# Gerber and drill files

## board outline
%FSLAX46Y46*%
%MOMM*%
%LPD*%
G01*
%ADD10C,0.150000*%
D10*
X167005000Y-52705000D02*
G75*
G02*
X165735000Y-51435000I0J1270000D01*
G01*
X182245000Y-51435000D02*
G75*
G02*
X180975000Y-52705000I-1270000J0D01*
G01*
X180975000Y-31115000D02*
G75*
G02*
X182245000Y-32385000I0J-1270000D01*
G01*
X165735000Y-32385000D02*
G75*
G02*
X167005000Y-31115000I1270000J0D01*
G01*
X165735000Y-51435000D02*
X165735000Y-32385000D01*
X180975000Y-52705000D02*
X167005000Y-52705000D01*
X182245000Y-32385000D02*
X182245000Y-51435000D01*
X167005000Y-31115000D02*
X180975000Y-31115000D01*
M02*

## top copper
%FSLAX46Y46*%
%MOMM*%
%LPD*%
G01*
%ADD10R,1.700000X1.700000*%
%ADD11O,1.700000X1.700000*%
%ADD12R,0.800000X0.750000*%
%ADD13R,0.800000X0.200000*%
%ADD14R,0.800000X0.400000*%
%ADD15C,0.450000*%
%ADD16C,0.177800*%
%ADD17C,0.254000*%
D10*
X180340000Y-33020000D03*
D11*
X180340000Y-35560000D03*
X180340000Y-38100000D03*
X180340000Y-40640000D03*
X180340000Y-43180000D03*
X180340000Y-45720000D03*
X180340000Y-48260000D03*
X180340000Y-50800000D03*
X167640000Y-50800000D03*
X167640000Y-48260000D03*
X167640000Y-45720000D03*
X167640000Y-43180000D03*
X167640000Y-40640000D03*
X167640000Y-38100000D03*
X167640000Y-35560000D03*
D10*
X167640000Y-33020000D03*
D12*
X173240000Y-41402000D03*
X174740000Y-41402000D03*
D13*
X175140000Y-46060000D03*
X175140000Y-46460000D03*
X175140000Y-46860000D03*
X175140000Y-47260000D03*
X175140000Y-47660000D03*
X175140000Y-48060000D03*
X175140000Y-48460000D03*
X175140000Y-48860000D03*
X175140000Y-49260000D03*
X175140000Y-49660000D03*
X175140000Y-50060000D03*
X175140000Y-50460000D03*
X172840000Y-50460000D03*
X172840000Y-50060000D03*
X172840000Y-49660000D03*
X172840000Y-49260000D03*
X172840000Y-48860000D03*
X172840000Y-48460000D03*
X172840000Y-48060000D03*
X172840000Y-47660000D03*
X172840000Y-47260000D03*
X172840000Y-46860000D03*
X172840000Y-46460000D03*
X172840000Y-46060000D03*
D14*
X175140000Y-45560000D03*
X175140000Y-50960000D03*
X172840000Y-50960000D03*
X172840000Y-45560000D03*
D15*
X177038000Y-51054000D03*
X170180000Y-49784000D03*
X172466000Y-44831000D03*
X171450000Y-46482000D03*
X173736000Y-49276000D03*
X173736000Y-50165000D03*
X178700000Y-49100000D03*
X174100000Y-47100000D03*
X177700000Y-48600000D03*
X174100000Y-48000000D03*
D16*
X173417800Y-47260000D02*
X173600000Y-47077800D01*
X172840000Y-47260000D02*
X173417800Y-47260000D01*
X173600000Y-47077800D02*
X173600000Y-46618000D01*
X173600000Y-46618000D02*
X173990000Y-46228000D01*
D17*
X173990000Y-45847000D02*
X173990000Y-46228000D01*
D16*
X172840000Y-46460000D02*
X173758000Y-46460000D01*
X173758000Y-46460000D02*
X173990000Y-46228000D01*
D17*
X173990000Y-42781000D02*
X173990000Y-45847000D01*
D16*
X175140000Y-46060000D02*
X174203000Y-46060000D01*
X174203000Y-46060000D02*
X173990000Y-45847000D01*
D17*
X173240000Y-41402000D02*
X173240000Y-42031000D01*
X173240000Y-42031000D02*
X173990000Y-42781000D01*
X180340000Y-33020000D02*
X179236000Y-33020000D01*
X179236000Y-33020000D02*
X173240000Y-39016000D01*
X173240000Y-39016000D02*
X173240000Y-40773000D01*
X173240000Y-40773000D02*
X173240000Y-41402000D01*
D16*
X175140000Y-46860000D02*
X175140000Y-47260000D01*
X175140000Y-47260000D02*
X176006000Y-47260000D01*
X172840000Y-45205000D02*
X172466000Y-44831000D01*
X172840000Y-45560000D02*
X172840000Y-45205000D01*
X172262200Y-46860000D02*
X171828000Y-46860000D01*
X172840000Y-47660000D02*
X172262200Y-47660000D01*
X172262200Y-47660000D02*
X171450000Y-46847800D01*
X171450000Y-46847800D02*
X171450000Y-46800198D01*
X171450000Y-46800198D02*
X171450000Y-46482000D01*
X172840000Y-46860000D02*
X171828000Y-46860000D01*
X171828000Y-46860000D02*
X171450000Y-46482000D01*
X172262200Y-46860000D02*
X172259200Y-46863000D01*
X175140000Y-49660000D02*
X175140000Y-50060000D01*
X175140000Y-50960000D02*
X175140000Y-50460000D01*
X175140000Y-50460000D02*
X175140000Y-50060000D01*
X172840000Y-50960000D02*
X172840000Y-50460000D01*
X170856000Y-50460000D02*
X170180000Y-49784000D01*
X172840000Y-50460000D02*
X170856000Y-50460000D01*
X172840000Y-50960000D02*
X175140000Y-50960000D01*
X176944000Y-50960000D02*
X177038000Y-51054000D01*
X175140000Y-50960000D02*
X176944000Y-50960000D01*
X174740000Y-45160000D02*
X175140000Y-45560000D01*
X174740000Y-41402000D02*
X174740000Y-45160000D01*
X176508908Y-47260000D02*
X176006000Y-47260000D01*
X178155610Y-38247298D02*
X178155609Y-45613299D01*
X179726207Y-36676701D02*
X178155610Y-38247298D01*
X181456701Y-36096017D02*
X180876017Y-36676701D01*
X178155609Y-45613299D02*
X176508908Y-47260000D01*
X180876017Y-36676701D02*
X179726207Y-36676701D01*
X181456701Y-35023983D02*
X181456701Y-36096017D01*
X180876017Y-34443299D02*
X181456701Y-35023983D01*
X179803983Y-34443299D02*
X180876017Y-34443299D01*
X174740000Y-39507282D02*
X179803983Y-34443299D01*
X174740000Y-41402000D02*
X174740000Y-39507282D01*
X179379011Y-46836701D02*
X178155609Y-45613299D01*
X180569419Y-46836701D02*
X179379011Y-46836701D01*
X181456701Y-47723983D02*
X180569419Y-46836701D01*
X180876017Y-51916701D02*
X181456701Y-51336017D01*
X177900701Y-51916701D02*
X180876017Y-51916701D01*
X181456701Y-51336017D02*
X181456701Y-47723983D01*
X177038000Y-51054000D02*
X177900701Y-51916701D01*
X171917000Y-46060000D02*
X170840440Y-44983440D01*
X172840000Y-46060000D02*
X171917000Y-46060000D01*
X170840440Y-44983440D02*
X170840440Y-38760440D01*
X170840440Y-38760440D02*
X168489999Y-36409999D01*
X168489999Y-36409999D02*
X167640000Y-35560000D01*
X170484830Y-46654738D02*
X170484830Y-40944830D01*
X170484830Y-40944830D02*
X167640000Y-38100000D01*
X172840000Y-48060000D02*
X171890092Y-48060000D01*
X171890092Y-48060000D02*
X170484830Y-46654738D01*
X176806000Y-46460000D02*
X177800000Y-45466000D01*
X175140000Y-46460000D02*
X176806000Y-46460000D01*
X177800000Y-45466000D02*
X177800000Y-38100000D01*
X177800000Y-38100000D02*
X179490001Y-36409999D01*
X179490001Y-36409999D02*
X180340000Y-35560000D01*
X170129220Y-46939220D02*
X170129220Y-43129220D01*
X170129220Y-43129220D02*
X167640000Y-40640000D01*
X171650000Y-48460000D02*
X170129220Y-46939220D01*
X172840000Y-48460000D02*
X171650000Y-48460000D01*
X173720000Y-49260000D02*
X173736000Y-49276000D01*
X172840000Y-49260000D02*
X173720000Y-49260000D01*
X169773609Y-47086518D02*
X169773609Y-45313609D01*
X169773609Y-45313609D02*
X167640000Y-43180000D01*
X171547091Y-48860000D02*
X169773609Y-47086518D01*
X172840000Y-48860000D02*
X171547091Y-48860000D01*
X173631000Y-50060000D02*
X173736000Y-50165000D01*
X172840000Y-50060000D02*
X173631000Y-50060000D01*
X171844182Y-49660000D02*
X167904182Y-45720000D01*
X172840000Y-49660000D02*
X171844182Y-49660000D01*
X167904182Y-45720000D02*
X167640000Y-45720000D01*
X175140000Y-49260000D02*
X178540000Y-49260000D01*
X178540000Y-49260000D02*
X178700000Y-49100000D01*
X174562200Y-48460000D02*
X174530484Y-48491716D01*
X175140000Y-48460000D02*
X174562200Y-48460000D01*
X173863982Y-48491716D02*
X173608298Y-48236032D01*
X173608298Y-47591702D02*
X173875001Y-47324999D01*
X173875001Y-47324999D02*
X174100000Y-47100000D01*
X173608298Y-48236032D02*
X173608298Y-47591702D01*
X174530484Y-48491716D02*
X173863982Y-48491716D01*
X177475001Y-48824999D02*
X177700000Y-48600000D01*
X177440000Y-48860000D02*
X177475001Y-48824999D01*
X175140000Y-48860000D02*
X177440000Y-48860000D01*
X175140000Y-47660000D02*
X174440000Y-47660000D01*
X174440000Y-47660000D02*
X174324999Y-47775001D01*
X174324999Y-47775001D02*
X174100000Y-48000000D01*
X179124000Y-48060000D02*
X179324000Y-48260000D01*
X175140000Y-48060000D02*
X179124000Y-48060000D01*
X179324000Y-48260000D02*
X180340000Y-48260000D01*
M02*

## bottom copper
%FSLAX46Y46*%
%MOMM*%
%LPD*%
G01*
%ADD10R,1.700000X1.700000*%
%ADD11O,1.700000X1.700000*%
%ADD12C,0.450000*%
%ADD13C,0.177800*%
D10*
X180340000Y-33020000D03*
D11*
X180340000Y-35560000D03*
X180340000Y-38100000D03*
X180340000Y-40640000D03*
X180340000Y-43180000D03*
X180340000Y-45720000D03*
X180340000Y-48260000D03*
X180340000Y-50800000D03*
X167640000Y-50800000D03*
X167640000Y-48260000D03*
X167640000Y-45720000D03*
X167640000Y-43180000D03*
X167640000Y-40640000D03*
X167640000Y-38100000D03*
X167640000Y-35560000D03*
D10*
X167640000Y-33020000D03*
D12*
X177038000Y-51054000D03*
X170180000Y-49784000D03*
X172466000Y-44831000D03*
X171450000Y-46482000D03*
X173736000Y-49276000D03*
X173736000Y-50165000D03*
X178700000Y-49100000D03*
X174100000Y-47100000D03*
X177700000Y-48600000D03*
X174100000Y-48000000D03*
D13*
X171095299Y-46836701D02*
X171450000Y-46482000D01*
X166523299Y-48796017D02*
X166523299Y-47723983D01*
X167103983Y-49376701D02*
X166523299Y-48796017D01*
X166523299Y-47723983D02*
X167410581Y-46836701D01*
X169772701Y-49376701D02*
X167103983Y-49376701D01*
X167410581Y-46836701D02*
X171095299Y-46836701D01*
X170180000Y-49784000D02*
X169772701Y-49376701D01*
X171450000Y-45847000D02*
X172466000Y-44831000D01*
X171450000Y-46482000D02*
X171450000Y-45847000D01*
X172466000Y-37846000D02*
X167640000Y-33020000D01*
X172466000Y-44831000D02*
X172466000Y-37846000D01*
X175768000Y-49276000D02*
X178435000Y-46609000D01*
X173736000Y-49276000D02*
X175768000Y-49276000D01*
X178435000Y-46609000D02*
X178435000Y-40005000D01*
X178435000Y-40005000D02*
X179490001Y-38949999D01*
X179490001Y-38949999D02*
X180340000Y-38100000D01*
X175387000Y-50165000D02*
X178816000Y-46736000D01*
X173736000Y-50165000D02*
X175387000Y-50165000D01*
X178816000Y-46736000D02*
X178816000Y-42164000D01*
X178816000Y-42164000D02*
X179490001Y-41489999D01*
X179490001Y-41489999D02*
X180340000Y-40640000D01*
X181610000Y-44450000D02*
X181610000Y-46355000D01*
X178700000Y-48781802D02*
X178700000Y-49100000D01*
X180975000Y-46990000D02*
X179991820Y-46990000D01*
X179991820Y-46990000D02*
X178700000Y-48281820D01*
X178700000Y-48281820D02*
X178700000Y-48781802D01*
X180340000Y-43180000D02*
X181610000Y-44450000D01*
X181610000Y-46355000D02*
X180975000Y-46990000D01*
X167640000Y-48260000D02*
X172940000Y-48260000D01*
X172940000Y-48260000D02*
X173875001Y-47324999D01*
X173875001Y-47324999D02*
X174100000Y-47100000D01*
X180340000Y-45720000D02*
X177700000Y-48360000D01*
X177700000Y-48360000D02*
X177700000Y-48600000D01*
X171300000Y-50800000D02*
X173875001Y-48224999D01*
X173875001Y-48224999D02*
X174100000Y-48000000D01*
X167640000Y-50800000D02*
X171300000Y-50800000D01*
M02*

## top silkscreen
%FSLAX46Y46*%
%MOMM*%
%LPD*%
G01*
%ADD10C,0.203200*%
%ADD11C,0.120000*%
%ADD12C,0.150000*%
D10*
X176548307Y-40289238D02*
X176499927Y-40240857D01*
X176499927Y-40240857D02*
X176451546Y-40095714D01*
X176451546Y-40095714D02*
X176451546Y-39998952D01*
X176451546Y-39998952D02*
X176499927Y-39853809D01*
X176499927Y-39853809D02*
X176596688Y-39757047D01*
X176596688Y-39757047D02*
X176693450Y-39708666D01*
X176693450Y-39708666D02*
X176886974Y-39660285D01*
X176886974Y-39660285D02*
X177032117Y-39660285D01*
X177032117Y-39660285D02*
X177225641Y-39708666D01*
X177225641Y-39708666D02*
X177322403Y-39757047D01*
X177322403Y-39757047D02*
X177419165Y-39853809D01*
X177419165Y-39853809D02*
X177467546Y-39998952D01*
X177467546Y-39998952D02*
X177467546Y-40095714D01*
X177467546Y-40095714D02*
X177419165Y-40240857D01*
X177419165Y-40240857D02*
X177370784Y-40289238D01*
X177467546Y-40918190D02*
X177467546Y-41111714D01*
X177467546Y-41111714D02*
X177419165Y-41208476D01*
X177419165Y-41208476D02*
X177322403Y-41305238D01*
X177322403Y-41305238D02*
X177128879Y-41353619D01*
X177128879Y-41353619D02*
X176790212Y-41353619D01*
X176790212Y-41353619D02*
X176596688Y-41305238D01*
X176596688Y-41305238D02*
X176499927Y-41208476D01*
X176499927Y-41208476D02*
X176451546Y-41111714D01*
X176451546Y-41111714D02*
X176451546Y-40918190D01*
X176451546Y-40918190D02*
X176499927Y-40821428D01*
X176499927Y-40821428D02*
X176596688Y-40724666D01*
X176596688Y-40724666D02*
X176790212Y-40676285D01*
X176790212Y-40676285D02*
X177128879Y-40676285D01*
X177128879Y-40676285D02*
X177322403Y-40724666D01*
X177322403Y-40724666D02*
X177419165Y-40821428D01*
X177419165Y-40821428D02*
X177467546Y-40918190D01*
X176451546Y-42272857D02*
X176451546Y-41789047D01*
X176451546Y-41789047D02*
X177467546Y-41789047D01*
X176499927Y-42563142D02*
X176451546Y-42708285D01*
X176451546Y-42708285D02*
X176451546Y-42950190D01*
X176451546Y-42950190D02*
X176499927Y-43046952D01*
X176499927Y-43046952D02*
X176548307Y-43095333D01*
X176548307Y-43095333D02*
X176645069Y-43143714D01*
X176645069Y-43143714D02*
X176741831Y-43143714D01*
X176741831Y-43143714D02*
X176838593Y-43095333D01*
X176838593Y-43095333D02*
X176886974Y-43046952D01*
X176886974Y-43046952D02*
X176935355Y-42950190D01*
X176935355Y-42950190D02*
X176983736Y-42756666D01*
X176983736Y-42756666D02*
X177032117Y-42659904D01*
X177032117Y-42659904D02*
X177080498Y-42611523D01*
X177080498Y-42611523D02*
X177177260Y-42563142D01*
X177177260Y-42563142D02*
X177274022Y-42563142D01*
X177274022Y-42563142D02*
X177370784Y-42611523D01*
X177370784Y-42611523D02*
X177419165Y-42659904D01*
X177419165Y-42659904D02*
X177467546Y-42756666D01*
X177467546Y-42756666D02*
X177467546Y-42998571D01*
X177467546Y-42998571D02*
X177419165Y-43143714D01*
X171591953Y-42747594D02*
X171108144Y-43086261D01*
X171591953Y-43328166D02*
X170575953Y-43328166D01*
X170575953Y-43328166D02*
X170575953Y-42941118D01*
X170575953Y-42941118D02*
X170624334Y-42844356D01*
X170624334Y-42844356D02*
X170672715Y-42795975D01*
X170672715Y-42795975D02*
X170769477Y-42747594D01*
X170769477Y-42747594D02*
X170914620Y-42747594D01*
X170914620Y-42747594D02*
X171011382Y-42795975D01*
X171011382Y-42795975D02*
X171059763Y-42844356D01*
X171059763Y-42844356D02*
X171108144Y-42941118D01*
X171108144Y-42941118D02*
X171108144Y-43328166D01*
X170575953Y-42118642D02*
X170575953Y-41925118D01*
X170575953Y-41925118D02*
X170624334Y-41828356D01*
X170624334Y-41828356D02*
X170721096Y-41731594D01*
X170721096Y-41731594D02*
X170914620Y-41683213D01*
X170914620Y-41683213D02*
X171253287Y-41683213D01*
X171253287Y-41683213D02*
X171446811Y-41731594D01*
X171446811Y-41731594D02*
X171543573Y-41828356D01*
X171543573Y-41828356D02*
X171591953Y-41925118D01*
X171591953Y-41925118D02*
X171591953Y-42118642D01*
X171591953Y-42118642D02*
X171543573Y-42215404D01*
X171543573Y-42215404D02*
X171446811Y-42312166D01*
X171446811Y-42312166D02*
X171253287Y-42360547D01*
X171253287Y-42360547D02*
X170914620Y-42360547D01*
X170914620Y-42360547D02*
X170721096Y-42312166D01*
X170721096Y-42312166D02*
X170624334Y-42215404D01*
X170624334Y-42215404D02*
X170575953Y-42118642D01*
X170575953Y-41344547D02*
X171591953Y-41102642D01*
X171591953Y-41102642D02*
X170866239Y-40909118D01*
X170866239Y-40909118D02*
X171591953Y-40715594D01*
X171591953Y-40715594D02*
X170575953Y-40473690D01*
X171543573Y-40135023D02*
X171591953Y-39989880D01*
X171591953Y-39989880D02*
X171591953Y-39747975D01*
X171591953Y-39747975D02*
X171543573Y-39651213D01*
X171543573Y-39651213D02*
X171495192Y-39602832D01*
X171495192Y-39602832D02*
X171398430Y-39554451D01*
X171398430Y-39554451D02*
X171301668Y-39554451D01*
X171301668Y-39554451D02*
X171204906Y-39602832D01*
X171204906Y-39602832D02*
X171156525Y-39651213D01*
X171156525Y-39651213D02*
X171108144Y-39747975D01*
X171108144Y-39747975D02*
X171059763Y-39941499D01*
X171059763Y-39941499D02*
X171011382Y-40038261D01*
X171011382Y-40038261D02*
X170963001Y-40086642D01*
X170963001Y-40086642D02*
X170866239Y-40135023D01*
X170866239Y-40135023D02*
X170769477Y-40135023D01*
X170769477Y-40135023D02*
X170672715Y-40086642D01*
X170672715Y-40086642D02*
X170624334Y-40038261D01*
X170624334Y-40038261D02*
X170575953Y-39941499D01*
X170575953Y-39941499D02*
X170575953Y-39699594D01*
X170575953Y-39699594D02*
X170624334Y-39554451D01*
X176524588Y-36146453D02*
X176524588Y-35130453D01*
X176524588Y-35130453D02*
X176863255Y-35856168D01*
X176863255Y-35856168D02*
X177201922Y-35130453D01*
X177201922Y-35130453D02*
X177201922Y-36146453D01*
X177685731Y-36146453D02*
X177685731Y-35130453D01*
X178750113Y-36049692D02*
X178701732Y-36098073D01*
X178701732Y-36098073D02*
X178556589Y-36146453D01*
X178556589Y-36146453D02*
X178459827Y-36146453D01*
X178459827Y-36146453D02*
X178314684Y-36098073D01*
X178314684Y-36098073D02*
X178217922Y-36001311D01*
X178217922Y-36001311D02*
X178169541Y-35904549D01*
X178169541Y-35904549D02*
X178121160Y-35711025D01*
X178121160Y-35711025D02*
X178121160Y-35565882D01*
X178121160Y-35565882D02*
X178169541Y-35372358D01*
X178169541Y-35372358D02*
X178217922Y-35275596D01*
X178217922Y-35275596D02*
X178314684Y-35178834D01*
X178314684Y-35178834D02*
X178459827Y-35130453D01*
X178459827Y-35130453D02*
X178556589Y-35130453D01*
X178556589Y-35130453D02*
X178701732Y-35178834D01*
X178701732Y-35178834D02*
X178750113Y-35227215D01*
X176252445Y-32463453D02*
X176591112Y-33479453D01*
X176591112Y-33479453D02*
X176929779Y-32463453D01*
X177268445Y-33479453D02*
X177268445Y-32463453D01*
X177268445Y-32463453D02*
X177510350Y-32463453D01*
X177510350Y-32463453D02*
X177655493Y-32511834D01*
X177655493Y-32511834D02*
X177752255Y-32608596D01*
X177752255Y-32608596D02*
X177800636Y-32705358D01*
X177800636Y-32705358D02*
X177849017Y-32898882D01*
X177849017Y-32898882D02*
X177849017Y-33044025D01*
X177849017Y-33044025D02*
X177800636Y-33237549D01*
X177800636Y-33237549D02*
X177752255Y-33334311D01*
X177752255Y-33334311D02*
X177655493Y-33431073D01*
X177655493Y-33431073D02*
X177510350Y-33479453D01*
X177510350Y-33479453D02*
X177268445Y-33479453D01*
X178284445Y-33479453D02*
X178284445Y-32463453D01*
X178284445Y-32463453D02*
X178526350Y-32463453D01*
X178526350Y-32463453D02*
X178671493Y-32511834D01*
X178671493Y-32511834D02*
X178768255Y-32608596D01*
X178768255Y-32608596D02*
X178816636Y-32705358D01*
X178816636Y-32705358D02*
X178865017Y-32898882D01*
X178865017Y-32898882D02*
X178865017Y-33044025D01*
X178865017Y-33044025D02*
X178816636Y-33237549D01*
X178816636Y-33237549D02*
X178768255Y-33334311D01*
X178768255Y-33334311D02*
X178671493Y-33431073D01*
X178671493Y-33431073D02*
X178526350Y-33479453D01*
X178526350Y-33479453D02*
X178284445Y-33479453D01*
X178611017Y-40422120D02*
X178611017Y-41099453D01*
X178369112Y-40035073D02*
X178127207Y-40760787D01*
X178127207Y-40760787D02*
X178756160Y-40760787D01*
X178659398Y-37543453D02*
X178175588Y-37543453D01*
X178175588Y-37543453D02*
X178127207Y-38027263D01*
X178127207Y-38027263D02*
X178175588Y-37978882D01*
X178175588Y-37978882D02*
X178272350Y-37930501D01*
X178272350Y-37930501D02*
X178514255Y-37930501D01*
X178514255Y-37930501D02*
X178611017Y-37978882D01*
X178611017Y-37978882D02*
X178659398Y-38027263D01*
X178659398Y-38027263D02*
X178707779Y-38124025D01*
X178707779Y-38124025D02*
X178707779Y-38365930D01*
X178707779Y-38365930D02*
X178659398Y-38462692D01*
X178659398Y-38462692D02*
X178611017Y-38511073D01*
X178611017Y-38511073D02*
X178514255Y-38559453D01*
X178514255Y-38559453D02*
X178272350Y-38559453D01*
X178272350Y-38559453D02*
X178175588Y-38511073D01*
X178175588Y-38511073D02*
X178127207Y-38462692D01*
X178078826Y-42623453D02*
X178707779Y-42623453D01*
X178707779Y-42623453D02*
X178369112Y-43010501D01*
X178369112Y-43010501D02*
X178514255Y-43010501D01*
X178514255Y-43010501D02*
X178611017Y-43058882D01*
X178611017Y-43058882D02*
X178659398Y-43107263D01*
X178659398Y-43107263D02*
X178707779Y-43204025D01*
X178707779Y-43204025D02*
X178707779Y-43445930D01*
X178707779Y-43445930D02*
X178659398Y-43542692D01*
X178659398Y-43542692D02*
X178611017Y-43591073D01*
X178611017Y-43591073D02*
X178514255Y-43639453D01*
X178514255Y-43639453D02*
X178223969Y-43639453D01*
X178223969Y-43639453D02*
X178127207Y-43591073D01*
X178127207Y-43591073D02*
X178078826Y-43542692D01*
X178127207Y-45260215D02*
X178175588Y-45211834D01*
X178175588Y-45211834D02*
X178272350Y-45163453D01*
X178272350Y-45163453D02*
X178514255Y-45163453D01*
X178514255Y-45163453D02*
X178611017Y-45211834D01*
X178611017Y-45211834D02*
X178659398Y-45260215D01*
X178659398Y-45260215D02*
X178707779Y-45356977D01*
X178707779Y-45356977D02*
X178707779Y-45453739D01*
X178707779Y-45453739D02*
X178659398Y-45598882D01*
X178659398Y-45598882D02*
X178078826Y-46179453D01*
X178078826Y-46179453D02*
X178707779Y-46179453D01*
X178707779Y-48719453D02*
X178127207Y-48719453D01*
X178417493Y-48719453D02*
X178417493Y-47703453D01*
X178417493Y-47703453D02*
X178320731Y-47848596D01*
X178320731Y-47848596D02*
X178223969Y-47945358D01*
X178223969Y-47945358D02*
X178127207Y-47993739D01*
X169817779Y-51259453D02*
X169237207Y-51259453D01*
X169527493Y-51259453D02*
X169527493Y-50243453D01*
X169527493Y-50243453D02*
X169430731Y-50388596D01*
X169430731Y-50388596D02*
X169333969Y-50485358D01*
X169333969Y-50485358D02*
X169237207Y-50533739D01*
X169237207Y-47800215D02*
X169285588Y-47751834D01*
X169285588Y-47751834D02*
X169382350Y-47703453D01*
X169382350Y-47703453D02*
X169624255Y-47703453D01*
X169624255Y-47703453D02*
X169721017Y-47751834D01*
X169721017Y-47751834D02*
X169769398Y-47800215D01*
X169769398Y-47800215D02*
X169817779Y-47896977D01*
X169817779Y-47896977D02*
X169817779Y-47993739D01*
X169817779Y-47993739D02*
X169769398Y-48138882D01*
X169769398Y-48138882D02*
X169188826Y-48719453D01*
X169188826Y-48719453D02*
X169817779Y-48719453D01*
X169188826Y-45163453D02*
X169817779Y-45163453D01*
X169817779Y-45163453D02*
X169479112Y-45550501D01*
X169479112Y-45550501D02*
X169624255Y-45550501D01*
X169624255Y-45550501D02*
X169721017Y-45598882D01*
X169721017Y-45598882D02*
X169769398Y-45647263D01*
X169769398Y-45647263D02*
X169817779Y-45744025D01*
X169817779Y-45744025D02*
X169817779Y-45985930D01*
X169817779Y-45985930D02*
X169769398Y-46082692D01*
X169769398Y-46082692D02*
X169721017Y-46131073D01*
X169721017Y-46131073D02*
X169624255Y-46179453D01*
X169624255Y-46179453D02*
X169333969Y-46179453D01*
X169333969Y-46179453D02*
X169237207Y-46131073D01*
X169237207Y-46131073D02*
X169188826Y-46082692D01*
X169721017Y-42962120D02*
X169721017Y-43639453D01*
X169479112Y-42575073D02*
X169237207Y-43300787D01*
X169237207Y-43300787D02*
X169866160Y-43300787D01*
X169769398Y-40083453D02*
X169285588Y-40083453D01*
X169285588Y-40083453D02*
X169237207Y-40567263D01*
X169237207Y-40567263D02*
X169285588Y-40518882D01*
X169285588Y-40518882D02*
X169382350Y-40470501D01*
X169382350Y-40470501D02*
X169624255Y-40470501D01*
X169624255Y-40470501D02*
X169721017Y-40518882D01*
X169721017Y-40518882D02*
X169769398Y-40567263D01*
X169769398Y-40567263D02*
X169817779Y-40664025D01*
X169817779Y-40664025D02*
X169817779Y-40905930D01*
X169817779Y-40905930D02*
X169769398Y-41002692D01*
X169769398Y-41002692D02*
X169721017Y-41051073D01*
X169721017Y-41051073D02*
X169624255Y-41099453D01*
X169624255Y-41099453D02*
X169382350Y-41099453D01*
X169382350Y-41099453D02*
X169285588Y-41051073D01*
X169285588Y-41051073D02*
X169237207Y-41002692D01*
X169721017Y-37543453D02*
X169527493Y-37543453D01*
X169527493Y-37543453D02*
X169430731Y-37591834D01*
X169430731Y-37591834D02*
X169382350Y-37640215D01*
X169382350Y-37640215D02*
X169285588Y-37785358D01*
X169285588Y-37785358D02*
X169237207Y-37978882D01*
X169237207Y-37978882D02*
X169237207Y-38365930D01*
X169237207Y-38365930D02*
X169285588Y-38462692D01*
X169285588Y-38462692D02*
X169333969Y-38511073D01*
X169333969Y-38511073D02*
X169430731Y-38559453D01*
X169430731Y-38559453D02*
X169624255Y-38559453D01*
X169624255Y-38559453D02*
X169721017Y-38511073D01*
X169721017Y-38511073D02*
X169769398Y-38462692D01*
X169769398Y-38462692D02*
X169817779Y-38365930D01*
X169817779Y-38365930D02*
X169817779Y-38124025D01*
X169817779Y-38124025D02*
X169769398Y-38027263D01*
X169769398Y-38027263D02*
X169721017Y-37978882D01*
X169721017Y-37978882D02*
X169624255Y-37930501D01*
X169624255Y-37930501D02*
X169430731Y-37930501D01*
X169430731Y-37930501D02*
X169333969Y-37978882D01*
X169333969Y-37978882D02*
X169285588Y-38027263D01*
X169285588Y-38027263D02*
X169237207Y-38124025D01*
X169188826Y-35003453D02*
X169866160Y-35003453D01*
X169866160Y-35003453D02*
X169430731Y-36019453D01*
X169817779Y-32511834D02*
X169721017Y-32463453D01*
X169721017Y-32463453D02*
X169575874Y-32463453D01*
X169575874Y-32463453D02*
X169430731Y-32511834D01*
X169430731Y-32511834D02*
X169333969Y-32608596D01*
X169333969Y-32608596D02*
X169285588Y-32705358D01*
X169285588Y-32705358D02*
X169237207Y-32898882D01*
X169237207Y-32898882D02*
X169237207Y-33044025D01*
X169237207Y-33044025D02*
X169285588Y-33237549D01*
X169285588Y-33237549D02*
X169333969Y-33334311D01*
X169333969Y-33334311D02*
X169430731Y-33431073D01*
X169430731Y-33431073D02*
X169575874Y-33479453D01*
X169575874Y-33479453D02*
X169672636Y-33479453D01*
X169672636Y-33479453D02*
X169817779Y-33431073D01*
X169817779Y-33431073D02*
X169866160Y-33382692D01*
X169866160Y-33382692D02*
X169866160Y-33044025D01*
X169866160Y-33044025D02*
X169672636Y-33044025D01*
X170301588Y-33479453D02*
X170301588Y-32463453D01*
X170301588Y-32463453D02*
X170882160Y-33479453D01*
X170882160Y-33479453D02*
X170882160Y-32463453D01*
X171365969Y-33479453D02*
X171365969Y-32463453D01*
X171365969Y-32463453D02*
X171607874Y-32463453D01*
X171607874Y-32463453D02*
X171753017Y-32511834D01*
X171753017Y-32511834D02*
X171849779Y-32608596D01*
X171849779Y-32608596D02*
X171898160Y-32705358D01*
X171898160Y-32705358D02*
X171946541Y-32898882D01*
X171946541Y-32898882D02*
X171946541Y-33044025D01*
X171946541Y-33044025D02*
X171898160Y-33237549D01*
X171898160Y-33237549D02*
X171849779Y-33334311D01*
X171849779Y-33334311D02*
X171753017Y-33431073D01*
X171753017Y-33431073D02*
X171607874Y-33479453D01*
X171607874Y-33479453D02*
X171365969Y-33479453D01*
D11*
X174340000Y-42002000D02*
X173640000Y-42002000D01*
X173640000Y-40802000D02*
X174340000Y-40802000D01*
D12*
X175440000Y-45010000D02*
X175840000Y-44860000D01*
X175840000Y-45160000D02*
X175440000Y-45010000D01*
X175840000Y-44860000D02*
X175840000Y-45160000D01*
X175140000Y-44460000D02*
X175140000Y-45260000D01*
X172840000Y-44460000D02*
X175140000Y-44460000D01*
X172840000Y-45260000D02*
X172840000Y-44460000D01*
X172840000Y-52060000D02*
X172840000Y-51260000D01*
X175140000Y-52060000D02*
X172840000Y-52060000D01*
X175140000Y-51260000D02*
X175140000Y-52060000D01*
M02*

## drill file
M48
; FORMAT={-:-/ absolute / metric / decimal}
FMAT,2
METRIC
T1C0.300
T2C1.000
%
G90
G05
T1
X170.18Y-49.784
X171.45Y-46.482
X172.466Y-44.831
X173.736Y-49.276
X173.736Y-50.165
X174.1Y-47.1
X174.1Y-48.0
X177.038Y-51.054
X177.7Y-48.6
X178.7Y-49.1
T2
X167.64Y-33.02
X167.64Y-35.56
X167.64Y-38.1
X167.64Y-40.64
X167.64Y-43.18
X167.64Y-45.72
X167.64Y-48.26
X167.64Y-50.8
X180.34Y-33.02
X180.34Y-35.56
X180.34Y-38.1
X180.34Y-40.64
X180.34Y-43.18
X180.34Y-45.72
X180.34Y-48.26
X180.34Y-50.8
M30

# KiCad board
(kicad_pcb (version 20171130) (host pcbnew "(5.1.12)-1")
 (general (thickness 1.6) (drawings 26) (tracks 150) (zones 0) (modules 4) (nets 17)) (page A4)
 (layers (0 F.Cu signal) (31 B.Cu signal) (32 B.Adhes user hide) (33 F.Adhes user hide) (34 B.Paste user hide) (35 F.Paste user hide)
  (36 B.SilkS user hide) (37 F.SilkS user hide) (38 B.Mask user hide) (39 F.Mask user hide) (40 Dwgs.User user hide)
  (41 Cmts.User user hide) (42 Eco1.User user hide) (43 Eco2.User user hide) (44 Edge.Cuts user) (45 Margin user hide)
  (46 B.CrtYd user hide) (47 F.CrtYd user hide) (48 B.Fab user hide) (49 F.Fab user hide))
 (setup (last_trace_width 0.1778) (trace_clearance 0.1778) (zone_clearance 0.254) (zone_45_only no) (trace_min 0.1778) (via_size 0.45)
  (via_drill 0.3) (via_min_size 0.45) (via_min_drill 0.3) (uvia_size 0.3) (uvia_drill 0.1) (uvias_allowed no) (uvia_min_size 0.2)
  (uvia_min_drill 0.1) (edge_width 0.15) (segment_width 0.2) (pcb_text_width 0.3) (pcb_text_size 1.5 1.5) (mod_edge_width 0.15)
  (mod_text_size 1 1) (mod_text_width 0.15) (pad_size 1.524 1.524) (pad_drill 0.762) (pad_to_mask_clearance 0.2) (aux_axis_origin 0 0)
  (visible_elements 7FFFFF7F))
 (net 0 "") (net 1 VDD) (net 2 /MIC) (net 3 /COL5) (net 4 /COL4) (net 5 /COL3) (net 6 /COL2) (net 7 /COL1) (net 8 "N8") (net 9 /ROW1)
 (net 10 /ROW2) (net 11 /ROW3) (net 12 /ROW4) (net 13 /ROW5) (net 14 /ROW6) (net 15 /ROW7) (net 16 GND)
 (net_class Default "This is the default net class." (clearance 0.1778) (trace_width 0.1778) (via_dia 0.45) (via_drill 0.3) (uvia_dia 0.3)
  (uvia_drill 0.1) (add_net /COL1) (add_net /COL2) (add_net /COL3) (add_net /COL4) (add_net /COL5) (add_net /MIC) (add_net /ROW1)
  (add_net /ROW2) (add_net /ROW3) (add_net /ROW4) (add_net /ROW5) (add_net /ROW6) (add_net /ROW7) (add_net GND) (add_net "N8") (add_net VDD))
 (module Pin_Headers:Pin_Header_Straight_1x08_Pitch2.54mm (layer B.Cu) (at 180.34 33.02 180)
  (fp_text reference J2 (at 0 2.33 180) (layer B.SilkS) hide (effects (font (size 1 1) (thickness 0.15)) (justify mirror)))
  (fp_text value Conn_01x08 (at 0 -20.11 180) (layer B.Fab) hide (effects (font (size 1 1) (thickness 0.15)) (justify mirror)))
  (pad 1 thru_hole rect (at 0 0 180) (size 1.7 1.7) (drill 1) (layers *.Cu *.Mask) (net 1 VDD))
  (pad 2 thru_hole oval (at 0 -2.54 180) (size 1.7 1.7) (drill 1) (layers *.Cu *.Mask) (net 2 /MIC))
  (pad 3 thru_hole oval (at 0 -5.08 180) (size 1.7 1.7) (drill 1) (layers *.Cu *.Mask) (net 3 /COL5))
  (pad 4 thru_hole oval (at 0 -7.62 180) (size 1.7 1.7) (drill 1) (layers *.Cu *.Mask) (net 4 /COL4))
  (pad 5 thru_hole oval (at 0 -10.16 180) (size 1.7 1.7) (drill 1) (layers *.Cu *.Mask) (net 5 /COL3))
  (pad 6 thru_hole oval (at 0 -12.7 180) (size 1.7 1.7) (drill 1) (layers *.Cu *.Mask) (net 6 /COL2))
  (pad 7 thru_hole oval (at 0 -15.24 180) (size 1.7 1.7) (drill 1) (layers *.Cu *.Mask) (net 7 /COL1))
  (pad 8 thru_hole oval (at 0 -17.78 180) (size 1.7 1.7) (drill 1) (layers *.Cu *.Mask) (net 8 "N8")))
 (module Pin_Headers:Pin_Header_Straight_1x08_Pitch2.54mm (layer B.Cu) (at 167.64 33.02 180)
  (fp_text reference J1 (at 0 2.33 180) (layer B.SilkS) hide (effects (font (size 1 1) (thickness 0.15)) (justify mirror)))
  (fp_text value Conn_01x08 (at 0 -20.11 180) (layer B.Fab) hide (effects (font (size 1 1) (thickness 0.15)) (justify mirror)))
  (pad 8 thru_hole oval (at 0 -17.78 180) (size 1.7 1.7) (drill 1) (layers *.Cu *.Mask) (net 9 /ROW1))
  (pad 7 thru_hole oval (at 0 -15.24 180) (size 1.7 1.7) (drill 1) (layers *.Cu *.Mask) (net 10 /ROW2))
  (pad 6 thru_hole oval (at 0 -12.7 180) (size 1.7 1.7) (drill 1) (layers *.Cu *.Mask) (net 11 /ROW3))
  (pad 5 thru_hole oval (at 0 -10.16 180) (size 1.7 1.7) (drill 1) (layers *.Cu *.Mask) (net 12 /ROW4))
  (pad 4 thru_hole oval (at 0 -7.62 180) (size 1.7 1.7) (drill 1) (layers *.Cu *.Mask) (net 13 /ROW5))
  (pad 3 thru_hole oval (at 0 -5.08 180) (size 1.7 1.7) (drill 1) (layers *.Cu *.Mask) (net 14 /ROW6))
  (pad 2 thru_hole oval (at 0 -2.54 180) (size 1.7 1.7) (drill 1) (layers *.Cu *.Mask) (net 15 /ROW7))
  (pad 1 thru_hole rect (at 0 0 180) (size 1.7 1.7) (drill 1) (layers *.Cu *.Mask) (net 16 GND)))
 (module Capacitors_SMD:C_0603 (layer F.Cu) (at 173.99 41.402)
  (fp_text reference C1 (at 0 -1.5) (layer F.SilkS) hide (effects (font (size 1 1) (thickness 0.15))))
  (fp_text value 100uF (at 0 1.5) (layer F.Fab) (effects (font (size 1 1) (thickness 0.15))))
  (fp_line (start 0.35 0.6) (end -0.35 0.6) (layer F.SilkS) (width 0.12))
  (fp_line (start -0.35 -0.6) (end 0.35 -0.6) (layer F.SilkS) (width 0.12))
  (pad 1 smd rect (at -0.75 0) (size 0.8 0.75) (layers F.Cu F.Paste F.Mask) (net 1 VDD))
  (pad 2 smd rect (at 0.75 0) (size 0.8 0.75) (layers F.Cu F.Paste F.Mask) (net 16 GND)))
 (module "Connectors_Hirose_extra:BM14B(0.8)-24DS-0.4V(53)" (layer F.Cu) (at 173.99 48.26 270)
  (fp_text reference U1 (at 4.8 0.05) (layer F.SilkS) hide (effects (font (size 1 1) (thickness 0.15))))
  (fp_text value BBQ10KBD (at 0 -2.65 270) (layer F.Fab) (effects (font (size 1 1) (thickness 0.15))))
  (fp_line (start -3.25 -1.45) (end -3.4 -1.85) (layer F.SilkS) (width 0.15))
  (fp_line (start -3.1 -1.85) (end -3.25 -1.45) (layer F.SilkS) (width 0.15))
  (fp_line (start -3.4 -1.85) (end -3.1 -1.85) (layer F.SilkS) (width 0.15))
  (fp_line (start -3.8 -1.15) (end -3 -1.15) (layer F.SilkS) (width 0.15))
  (fp_line (start -3.8 1.15) (end -3.8 -1.15) (layer F.SilkS) (width 0.15))
  (fp_line (start -3 1.15) (end -3.8 1.15) (layer F.SilkS) (width 0.15))
  (fp_line (start 3.8 1.15) (end 3 1.15) (layer F.SilkS) (width 0.15))
  (fp_line (start 3.8 -1.15) (end 3.8 1.15) (layer F.SilkS) (width 0.15))
  (fp_line (start 3 -1.15) (end 3.8 -1.15) (layer F.SilkS) (width 0.15))
  (pad 2 smd rect (at -2.2 -1.15 270) (size 0.2 0.8) (layers F.Cu F.Paste F.Mask) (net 1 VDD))
  (pad 3 smd rect (at -1.8 -1.15 270) (size 0.2 0.8) (layers F.Cu F.Paste F.Mask) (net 2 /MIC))
  (pad 4 smd rect (at -1.4 -1.15 270) (size 0.2 0.8) (layers F.Cu F.Paste F.Mask) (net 16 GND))
  (pad 5 smd rect (at -1 -1.15 270) (size 0.2 0.8) (layers F.Cu F.Paste F.Mask) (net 16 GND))
  (pad 6 smd rect (at -0.6 -1.15 270) (size 0.2 0.8) (layers F.Cu F.Paste F.Mask) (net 9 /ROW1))
  (pad 7 smd rect (at -0.2 -1.15 270) (size 0.2 0.8) (layers F.Cu F.Paste F.Mask) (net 7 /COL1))
  (pad 8 smd rect (at 0.2 -1.15 270) (size 0.2 0.8) (layers F.Cu F.Paste F.Mask) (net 10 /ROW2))
  (pad 9 smd rect (at 0.6 -1.15 270) (size 0.2 0.8) (layers F.Cu F.Paste F.Mask) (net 6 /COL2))
  (pad 10 smd rect (at 1 -1.15 270) (size 0.2 0.8) (layers F.Cu F.Paste F.Mask) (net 5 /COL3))
  (pad 11 smd rect (at 1.4 -1.15 270) (size 0.2 0.8) (layers F.Cu F.Paste F.Mask) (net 16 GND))
  (pad 12 smd rect (at 1.8 -1.15 270) (size 0.2 0.8) (layers F.Cu F.Paste F.Mask) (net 16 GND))
  (pad 13 smd rect (at 2.2 -1.15 270) (size 0.2 0.8) (layers F.Cu F.Paste F.Mask) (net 16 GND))
  (pad 16 smd rect (at 2.2 1.15 270) (size 0.2 0.8) (layers F.Cu F.Paste F.Mask) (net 16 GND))
  (pad 17 smd rect (at 1.8 1.15 270) (size 0.2 0.8) (layers F.Cu F.Paste F.Mask) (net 4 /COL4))
  (pad 18 smd rect (at 1.4 1.15 270) (size 0.2 0.8) (layers F.Cu F.Paste F.Mask) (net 11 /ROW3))
  (pad 19 smd rect (at 1 1.15 270) (size 0.2 0.8) (layers F.Cu F.Paste F.Mask) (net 3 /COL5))
  (pad 20 smd rect (at 0.6 1.15 270) (size 0.2 0.8) (layers F.Cu F.Paste F.Mask) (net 12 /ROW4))
  (pad 21 smd rect (at 0.2 1.15 270) (size 0.2 0.8) (layers F.Cu F.Paste F.Mask) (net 13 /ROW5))
  (pad 22 smd rect (at -0.2 1.15 270) (size 0.2 0.8) (layers F.Cu F.Paste F.Mask) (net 14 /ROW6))
  (pad 23 smd rect (at -0.6 1.15 270) (size 0.2 0.8) (layers F.Cu F.Paste F.Mask) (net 16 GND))
  (pad 24 smd rect (at -1 1.15 270) (size 0.2 0.8) (layers F.Cu F.Paste F.Mask) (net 1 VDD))
  (pad 25 smd rect (at -1.4 1.15 270) (size 0.2 0.8) (layers F.Cu F.Paste F.Mask) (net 16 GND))
  (pad 26 smd rect (at -1.8 1.15 270) (size 0.2 0.8) (layers F.Cu F.Paste F.Mask) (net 1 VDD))
  (pad 27 smd rect (at -2.2 1.15 270) (size 0.2 0.8) (layers F.Cu F.Paste F.Mask) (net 15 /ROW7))
  (pad 1 smd rect (at -2.7 -1.15 270) (size 0.4 0.8) (layers F.Cu F.Paste F.Mask) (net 16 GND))
  (pad 14 smd rect (at 2.7 -1.15 270) (size 0.4 0.8) (layers F.Cu F.Paste F.Mask) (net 16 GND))
  (pad 15 smd rect (at 2.7 1.15 270) (size 0.4 0.8) (layers F.Cu F.Paste F.Mask) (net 16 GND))
  (pad 28 smd rect (at -2.7 1.15 270) (size 0.4 0.8) (layers F.Cu F.Paste F.Mask) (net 16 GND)))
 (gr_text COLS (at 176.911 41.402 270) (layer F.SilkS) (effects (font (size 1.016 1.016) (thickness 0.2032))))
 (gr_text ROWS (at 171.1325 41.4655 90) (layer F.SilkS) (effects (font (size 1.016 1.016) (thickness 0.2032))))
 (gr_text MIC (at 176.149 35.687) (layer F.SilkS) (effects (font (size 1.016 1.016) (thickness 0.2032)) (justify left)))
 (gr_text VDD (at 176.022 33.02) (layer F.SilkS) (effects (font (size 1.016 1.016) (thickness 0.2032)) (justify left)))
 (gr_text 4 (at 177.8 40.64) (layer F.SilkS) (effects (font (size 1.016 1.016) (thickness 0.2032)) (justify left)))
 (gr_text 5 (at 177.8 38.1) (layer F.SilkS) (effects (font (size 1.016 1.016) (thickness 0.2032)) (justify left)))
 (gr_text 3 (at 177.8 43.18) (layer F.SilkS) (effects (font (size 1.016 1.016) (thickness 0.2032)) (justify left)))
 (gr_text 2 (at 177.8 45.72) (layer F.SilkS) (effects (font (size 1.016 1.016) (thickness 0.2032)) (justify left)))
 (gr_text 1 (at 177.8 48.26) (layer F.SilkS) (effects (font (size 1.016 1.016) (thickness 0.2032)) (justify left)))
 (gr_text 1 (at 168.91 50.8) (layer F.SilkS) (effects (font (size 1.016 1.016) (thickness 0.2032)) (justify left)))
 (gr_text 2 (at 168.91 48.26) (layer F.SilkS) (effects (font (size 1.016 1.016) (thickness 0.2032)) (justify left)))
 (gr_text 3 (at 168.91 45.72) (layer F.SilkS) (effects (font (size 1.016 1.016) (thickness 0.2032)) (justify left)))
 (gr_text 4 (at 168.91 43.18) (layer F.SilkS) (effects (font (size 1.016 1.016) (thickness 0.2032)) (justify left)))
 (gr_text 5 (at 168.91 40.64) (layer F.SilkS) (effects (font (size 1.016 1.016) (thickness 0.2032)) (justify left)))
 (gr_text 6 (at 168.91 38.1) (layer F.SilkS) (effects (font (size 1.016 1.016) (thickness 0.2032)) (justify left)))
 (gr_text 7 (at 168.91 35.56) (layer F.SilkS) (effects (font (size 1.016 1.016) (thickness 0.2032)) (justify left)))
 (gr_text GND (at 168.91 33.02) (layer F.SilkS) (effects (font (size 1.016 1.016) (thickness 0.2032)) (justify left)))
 (gr_arc (start 167.005 51.435) (end 165.735 51.435) (angle -90) (layer Edge.Cuts) (width 0.15))
 (gr_arc (start 180.975 51.435) (end 180.975 52.705) (angle -90) (layer Edge.Cuts) (width 0.15))
 (gr_arc (start 180.975 32.385) (end 182.245 32.385) (angle -90) (layer Edge.Cuts) (width 0.15))
 (gr_arc (start 167.005 32.385) (end 167.005 31.115) (angle -90) (layer Edge.Cuts) (width 0.15))
 (gr_line (start 165.735 51.435) (end 165.735 32.385) (layer Edge.Cuts) (width 0.15))
 (gr_line (start 180.975 52.705) (end 167.005 52.705) (layer Edge.Cuts) (width 0.15))
 (gr_line (start 182.245 32.385) (end 182.245 51.435) (layer Edge.Cuts) (width 0.15))
 (gr_line (start 167.005 31.115) (end 180.975 31.115) (layer Edge.Cuts) (width 0.15))
 (segment (start 173.4178 47.26) (end 173.6 47.0778) (width 0.1778) (layer F.Cu) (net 1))
 (segment (start 172.84 47.26) (end 173.4178 47.26) (width 0.1778) (layer F.Cu) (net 1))
 (segment (start 173.6 47.0778) (end 173.6 46.618) (width 0.1778) (layer F.Cu) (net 1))
 (segment (start 173.6 46.618) (end 173.99 46.228) (width 0.1778) (layer F.Cu) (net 1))
 (segment (start 173.99 45.847) (end 173.99 46.228) (width 0.254) (layer F.Cu) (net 1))
 (segment (start 172.84 46.46) (end 173.758 46.46) (width 0.1778) (layer F.Cu) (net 1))
 (segment (start 173.758 46.46) (end 173.99 46.228) (width 0.1778) (layer F.Cu) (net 1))
 (segment (start 173.99 42.781) (end 173.99 45.847) (width 0.254) (layer F.Cu) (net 1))
 (segment (start 175.14 46.06) (end 174.203 46.06) (width 0.1778) (layer F.Cu) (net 1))
 (segment (start 174.203 46.06) (end 173.99 45.847) (width 0.1778) (layer F.Cu) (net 1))
 (segment (start 173.24 41.402) (end 173.24 42.031) (width 0.254) (layer F.Cu) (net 1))
 (segment (start 173.24 42.031) (end 173.99 42.781) (width 0.254) (layer F.Cu) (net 1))
 (segment (start 180.34 33.02) (end 179.236 33.02) (width 0.254) (layer F.Cu) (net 1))
 (segment (start 179.236 33.02) (end 173.24 39.016) (width 0.254) (layer F.Cu) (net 1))
 (segment (start 173.24 39.016) (end 173.24 40.773) (width 0.254) (layer F.Cu) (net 1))
 (segment (start 173.24 40.773) (end 173.24 41.402) (width 0.254) (layer F.Cu) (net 1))
 (segment (start 175.14 46.86) (end 175.14 47.26) (width 0.1778) (layer F.Cu) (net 16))
 (segment (start 175.14 47.26) (end 176.006 47.26) (width 0.1778) (layer F.Cu) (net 16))
 (segment (start 172.84 45.205) (end 172.466 44.831) (width 0.1778) (layer F.Cu) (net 16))
 (segment (start 172.84 45.56) (end 172.84 45.205) (width 0.1778) (layer F.Cu) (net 16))
 (segment (start 172.2622 46.86) (end 171.828 46.86) (width 0.1778) (layer F.Cu) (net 16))
 (segment (start 172.84 47.66) (end 172.2622 47.66) (width 0.1778) (layer F.Cu) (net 16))
 (segment (start 172.2622 47.66) (end 171.45 46.8478) (width 0.1778) (layer F.Cu) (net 16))
 (segment (start 171.45 46.8478) (end 171.45 46.800198) (width 0.1778) (layer F.Cu) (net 16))
 (segment (start 171.45 46.800198) (end 171.45 46.482) (width 0.1778) (layer F.Cu) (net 16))
 (segment (start 172.84 46.86) (end 171.828 46.86) (width 0.1778) (layer F.Cu) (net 16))
 (segment (start 171.828 46.86) (end 171.45 46.482) (width 0.1778) (layer F.Cu) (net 16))
 (segment (start 172.2622 46.86) (end 172.2592 46.863) (width 0.1778) (layer F.Cu) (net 16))
 (segment (start 175.14 49.66) (end 175.14 50.06) (width 0.1778) (layer F.Cu) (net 16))
 (segment (start 175.14 50.96) (end 175.14 50.46) (width 0.1778) (layer F.Cu) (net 16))
 (segment (start 175.14 50.46) (end 175.14 50.06) (width 0.1778) (layer F.Cu) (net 16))
 (segment (start 172.84 50.96) (end 172.84 50.46) (width 0.1778) (layer F.Cu) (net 16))
 (segment (start 170.856 50.46) (end 170.18 49.784) (width 0.1778) (layer F.Cu) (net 16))
 (segment (start 172.84 50.46) (end 170.856 50.46) (width 0.1778) (layer F.Cu) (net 16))
 (segment (start 172.84 50.96) (end 175.14 50.96) (width 0.1778) (layer F.Cu) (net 16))
 (segment (start 176.944 50.96) (end 177.038 51.054) (width 0.1778) (layer F.Cu) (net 16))
 (segment (start 175.14 50.96) (end 176.944 50.96) (width 0.1778) (layer F.Cu) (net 16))
 (segment (start 171.095299 46.836701) (end 171.45 46.482) (width 0.1778) (layer B.Cu) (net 16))
 (segment (start 166.523299 48.796017) (end 166.523299 47.723983) (width 0.1778) (layer B.Cu) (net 16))
 (segment (start 167.103983 49.376701) (end 166.523299 48.796017) (width 0.1778) (layer B.Cu) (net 16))
 (segment (start 166.523299 47.723983) (end 167.410581 46.836701) (width 0.1778) (layer B.Cu) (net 16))
 (segment (start 169.772701 49.376701) (end 167.103983 49.376701) (width 0.1778) (layer B.Cu) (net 16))
 (segment (start 167.410581 46.836701) (end 171.095299 46.836701) (width 0.1778) (layer B.Cu) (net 16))
 (segment (start 170.18 49.784) (end 169.772701 49.376701) (width 0.1778) (layer B.Cu) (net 16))
 (segment (start 171.45 45.847) (end 172.466 44.831) (width 0.1778) (layer B.Cu) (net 16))
 (segment (start 171.45 46.482) (end 171.45 45.847) (width 0.1778) (layer B.Cu) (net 16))
 (segment (start 172.466 37.846) (end 167.64 33.02) (width 0.1778) (layer B.Cu) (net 16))
 (segment (start 172.466 44.831) (end 172.466 37.846) (width 0.1778) (layer B.Cu) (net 16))
 (segment (start 174.74 45.16) (end 175.14 45.56) (width 0.1778) (layer F.Cu) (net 16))
 (segment (start 174.74 41.402) (end 174.74 45.16) (width 0.1778) (layer F.Cu) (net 16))
 (segment (start 176.508908 47.26) (end 176.006 47.26) (width 0.1778) (layer F.Cu) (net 16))
 (segment (start 178.15561 38.247298) (end 178.155609 45.613299) (width 0.1778) (layer F.Cu) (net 16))
 (segment (start 179.726207 36.676701) (end 178.15561 38.247298) (width 0.1778) (layer F.Cu) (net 16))
 (segment (start 181.456701 36.096017) (end 180.876017 36.676701) (width 0.1778) (layer F.Cu) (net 16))
 (segment (start 178.155609 45.613299) (end 176.508908 47.26) (width 0.1778) (layer F.Cu) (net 16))
 (segment (start 180.876017 36.676701) (end 179.726207 36.676701) (width 0.1778) (layer F.Cu) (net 16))
 (segment (start 181.456701 35.023983) (end 181.456701 36.096017) (width 0.1778) (layer F.Cu) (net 16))
 (segment (start 180.876017 34.443299) (end 181.456701 35.023983) (width 0.1778) (layer F.Cu) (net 16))
 (segment (start 179.803983 34.443299) (end 180.876017 34.443299) (width 0.1778) (layer F.Cu) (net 16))
 (segment (start 174.74 39.507282) (end 179.803983 34.443299) (width 0.1778) (layer F.Cu) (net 16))
 (segment (start 174.74 41.402) (end 174.74 39.507282) (width 0.1778) (layer F.Cu) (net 16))
 (segment (start 179.379011 46.836701) (end 178.155609 45.613299) (width 0.1778) (layer F.Cu) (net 16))
 (segment (start 180.569419 46.836701) (end 179.379011 46.836701) (width 0.1778) (layer F.Cu) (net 16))
 (segment (start 181.456701 47.723983) (end 180.569419 46.836701) (width 0.1778) (layer F.Cu) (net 16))
 (segment (start 180.876017 51.916701) (end 181.456701 51.336017) (width 0.1778) (layer F.Cu) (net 16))
 (segment (start 177.900701 51.916701) (end 180.876017 51.916701) (width 0.1778) (layer F.Cu) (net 16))
 (segment (start 181.456701 51.336017) (end 181.456701 47.723983) (width 0.1778) (layer F.Cu) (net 16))
 (segment (start 177.038 51.054) (end 177.900701 51.916701) (width 0.1778) (layer F.Cu) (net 16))
 (segment (start 171.917 46.06) (end 170.84044 44.98344) (width 0.1778) (layer F.Cu) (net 15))
 (segment (start 172.84 46.06) (end 171.917 46.06) (width 0.1778) (layer F.Cu) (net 15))
 (segment (start 170.84044 44.98344) (end 170.84044 38.76044) (width 0.1778) (layer F.Cu) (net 15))
 (segment (start 170.84044 38.76044) (end 168.489999 36.409999) (width 0.1778) (layer F.Cu) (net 15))
 (segment (start 168.489999 36.409999) (end 167.64 35.56) (width 0.1778) (layer F.Cu) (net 15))
 (segment (start 170.48483 46.654738) (end 170.48483 40.94483) (width 0.1778) (layer F.Cu) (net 14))
 (segment (start 170.48483 40.94483) (end 167.64 38.1) (width 0.1778) (layer F.Cu) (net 14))
 (segment (start 172.84 48.06) (end 171.890092 48.06) (width 0.1778) (layer F.Cu) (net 14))
 (segment (start 171.890092 48.06) (end 170.48483 46.654738) (width 0.1778) (layer F.Cu) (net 14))
 (segment (start 176.806 46.46) (end 177.8 45.466) (width 0.1778) (layer F.Cu) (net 2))
 (segment (start 175.14 46.46) (end 176.806 46.46) (width 0.1778) (layer F.Cu) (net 2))
 (segment (start 177.8 45.466) (end 177.8 38.1) (width 0.1778) (layer F.Cu) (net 2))
 (segment (start 177.8 38.1) (end 179.490001 36.409999) (width 0.1778) (layer F.Cu) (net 2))
 (segment (start 179.490001 36.409999) (end 180.34 35.56) (width 0.1778) (layer F.Cu) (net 2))
 (segment (start 170.12922 46.93922) (end 170.12922 43.12922) (width 0.1778) (layer F.Cu) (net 13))
 (segment (start 170.12922 43.12922) (end 167.64 40.64) (width 0.1778) (layer F.Cu) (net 13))
 (segment (start 171.65 48.46) (end 170.12922 46.93922) (width 0.1778) (layer F.Cu) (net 13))
 (segment (start 172.84 48.46) (end 171.65 48.46) (width 0.1778) (layer F.Cu) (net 13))
 (segment (start 175.768 49.276) (end 178.435 46.609) (width 0.1778) (layer B.Cu) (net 3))
 (segment (start 173.736 49.276) (end 175.768 49.276) (width 0.1778) (layer B.Cu) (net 3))
 (segment (start 178.435 46.609) (end 178.435 40.005) (width 0.1778) (layer B.Cu) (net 3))
 (segment (start 178.435 40.005) (end 179.490001 38.949999) (width 0.1778) (layer B.Cu) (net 3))
 (segment (start 179.490001 38.949999) (end 180.34 38.1) (width 0.1778) (layer B.Cu) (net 3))
 (segment (start 173.72 49.26) (end 173.736 49.276) (width 0.1778) (layer F.Cu) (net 3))
 (segment (start 172.84 49.26) (end 173.72 49.26) (width 0.1778) (layer F.Cu) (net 3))
 (segment (start 169.773609 47.086518) (end 169.773609 45.313609) (width 0.1778) (layer F.Cu) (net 12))
 (segment (start 169.773609 45.313609) (end 167.64 43.18) (width 0.1778) (layer F.Cu) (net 12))
 (segment (start 171.547091 48.86) (end 169.773609 47.086518) (width 0.1778) (layer F.Cu) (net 12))
 (segment (start 172.84 48.86) (end 171.547091 48.86) (width 0.1778) (layer F.Cu) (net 12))
 (segment (start 175.387 50.165) (end 178.816 46.736) (width 0.1778) (layer B.Cu) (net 4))
 (segment (start 173.736 50.165) (end 175.387 50.165) (width 0.1778) (layer B.Cu) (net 4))
 (segment (start 178.816 46.736) (end 178.816 42.164) (width 0.1778) (layer B.Cu) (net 4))
 (segment (start 178.816 42.164) (end 179.490001 41.489999) (width 0.1778) (layer B.Cu) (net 4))
 (segment (start 179.490001 41.489999) (end 180.34 40.64) (width 0.1778) (layer B.Cu) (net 4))
 (segment (start 173.631 50.06) (end 173.736 50.165) (width 0.1778) (layer F.Cu) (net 4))
 (segment (start 172.84 50.06) (end 173.631 50.06) (width 0.1778) (layer F.Cu) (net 4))
 (segment (start 171.844182 49.66) (end 167.904182 45.72) (width 0.1778) (layer F.Cu) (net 11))
 (segment (start 172.84 49.66) (end 171.844182 49.66) (width 0.1778) (layer F.Cu) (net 11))
 (segment (start 167.904182 45.72) (end 167.64 45.72) (width 0.1778) (layer F.Cu) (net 11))
 (segment (start 181.61 44.45) (end 181.61 46.355) (width 0.1778) (layer B.Cu) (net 5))
 (segment (start 178.7 48.781802) (end 178.7 49.1) (width 0.1778) (layer B.Cu) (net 5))
 (segment (start 180.975 46.99) (end 179.99182 46.99) (width 0.1778) (layer B.Cu) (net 5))
 (segment (start 175.14 49.26) (end 178.54 49.26) (width 0.1778) (layer F.Cu) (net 5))
 (segment (start 178.54 49.26) (end 178.7 49.1) (width 0.1778) (layer F.Cu) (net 5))
 (segment (start 179.99182 46.99) (end 178.7 48.28182) (width 0.1778) (layer B.Cu) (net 5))
 (segment (start 178.7 48.28182) (end 178.7 48.781802) (width 0.1778) (layer B.Cu) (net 5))
 (segment (start 180.34 43.18) (end 181.61 44.45) (width 0.1778) (layer B.Cu) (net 5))
 (segment (start 181.61 46.355) (end 180.975 46.99) (width 0.1778) (layer B.Cu) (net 5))
 (segment (start 174.5622 48.46) (end 174.530484 48.491716) (width 0.1778) (layer F.Cu) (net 10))
 (segment (start 175.14 48.46) (end 174.5622 48.46) (width 0.1778) (layer F.Cu) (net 10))
 (segment (start 173.863982 48.491716) (end 173.608298 48.236032) (width 0.1778) (layer F.Cu) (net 10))
 (segment (start 173.608298 47.591702) (end 173.875001 47.324999) (width 0.1778) (layer F.Cu) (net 10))
 (segment (start 173.875001 47.324999) (end 174.1 47.1) (width 0.1778) (layer F.Cu) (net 10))
 (segment (start 173.608298 48.236032) (end 173.608298 47.591702) (width 0.1778) (layer F.Cu) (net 10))
 (segment (start 174.530484 48.491716) (end 173.863982 48.491716) (width 0.1778) (layer F.Cu) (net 10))
 (segment (start 167.64 48.26) (end 172.94 48.26) (width 0.1778) (layer B.Cu) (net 10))
 (segment (start 172.94 48.26) (end 173.875001 47.324999) (width 0.1778) (layer B.Cu) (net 10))
 (segment (start 173.875001 47.324999) (end 174.1 47.1) (width 0.1778) (layer B.Cu) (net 10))
 (segment (start 180.34 45.72) (end 177.7 48.36) (width 0.1778) (layer B.Cu) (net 6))
 (segment (start 177.7 48.36) (end 177.7 48.6) (width 0.1778) (layer B.Cu) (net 6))
 (segment (start 177.475001 48.824999) (end 177.7 48.6) (width 0.1778) (layer F.Cu) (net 6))
 (segment (start 177.44 48.86) (end 177.475001 48.824999) (width 0.1778) (layer F.Cu) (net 6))
 (segment (start 175.14 48.86) (end 177.44 48.86) (width 0.1778) (layer F.Cu) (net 6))
 (segment (start 175.14 47.66) (end 174.44 47.66) (width 0.1778) (layer F.Cu) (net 9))
 (segment (start 171.3 50.8) (end 173.875001 48.224999) (width 0.1778) (layer B.Cu) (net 9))
 (segment (start 174.44 47.66) (end 174.324999 47.775001) (width 0.1778) (layer F.Cu) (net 9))
 (segment (start 174.324999 47.775001) (end 174.1 48) (width 0.1778) (layer F.Cu) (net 9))
 (segment (start 173.875001 48.224999) (end 174.1 48) (width 0.1778) (layer B.Cu) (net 9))
 (segment (start 167.64 50.8) (end 171.3 50.8) (width 0.1778) (layer B.Cu) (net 9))
 (segment (start 179.124 48.06) (end 179.324 48.26) (width 0.1778) (layer F.Cu) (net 7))
 (segment (start 175.14 48.06) (end 179.124 48.06) (width 0.1778) (layer F.Cu) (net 7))
 (segment (start 179.324 48.26) (end 180.34 48.26) (width 0.1778) (layer F.Cu) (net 7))
 (via (at 177.038 51.054) (size 0.45) (drill 0.3) (layers F.Cu B.Cu) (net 16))
 (via (at 170.18 49.784) (size 0.45) (drill 0.3) (layers F.Cu B.Cu) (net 16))
 (via (at 172.466 44.831) (size 0.45) (drill 0.3) (layers F.Cu B.Cu) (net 16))
 (via (at 171.45 46.482) (size 0.45) (drill 0.3) (layers F.Cu B.Cu) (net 16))
 (via (at 173.736 49.276) (size 0.45) (drill 0.3) (layers F.Cu B.Cu) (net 3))
 (via (at 173.736 50.165) (size 0.45) (drill 0.3) (layers F.Cu B.Cu) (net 4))
 (via (at 178.7 49.1) (size 0.45) (drill 0.3) (layers F.Cu B.Cu) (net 5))
 (via (at 174.1 47.1) (size 0.45) (drill 0.3) (layers F.Cu B.Cu) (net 10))
 (via (at 177.7 48.6) (size 0.45) (drill 0.3) (layers F.Cu B.Cu) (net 6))
 (via (at 174.1 48) (size 0.45) (drill 0.3) (layers F.Cu B.Cu) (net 9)))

